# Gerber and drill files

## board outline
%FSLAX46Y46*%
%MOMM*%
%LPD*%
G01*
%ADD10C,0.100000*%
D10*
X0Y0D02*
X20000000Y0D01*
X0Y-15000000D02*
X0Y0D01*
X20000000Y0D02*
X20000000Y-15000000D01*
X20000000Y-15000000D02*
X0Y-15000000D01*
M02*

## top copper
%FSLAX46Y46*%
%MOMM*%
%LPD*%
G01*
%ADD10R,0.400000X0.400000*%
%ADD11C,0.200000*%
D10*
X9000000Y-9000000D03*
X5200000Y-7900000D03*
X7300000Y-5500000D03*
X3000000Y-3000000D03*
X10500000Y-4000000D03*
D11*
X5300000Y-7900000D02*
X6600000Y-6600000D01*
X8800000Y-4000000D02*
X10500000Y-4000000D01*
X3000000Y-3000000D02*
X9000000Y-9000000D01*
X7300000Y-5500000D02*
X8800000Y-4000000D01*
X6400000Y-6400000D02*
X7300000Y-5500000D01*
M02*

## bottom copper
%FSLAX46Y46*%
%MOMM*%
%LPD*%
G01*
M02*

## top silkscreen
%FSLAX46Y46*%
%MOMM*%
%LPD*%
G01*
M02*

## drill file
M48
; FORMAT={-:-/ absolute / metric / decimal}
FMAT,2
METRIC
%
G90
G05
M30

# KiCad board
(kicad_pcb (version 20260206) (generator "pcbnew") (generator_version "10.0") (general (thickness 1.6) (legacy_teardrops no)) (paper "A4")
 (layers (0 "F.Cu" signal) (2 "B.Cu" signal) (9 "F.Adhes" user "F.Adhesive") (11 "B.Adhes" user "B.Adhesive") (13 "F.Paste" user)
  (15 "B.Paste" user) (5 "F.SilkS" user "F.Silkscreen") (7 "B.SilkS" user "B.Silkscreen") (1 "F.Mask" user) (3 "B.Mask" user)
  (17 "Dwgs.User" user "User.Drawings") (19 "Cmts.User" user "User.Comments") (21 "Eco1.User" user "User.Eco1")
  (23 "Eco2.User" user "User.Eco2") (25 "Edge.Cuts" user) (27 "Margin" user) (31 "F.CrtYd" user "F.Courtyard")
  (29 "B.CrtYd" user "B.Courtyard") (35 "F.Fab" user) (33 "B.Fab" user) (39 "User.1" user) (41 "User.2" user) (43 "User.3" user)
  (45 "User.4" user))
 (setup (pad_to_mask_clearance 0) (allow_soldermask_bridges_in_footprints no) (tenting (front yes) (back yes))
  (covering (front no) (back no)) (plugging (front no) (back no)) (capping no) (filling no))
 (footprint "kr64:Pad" (layer "F.Cu") (at 9 9)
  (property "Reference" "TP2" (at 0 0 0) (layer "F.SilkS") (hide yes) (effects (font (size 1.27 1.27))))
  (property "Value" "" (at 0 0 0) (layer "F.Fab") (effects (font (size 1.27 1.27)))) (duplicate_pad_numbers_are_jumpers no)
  (pad "1" smd rect (at 0 0) (size 0.4 0.4) (layers "F.Cu" "F.Mask" "F.Paste") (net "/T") (thermal_bridge_angle 45)))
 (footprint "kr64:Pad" (layer "F.Cu") (at 5.2 7.9)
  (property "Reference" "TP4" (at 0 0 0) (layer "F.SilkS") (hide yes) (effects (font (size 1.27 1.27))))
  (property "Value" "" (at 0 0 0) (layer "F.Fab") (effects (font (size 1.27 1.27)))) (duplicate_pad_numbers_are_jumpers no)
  (pad "1" smd rect (at 0 0) (size 0.4 0.4) (layers "F.Cu" "F.Mask" "F.Paste") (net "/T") (thermal_bridge_angle 45)))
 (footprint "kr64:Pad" (layer "F.Cu") (at 7.3 5.5)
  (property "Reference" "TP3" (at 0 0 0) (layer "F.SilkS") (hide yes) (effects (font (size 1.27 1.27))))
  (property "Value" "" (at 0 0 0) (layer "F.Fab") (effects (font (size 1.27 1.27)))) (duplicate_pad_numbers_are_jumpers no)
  (pad "1" smd rect (at 0 0) (size 0.4 0.4) (layers "F.Cu" "F.Mask" "F.Paste") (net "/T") (thermal_bridge_angle 45)))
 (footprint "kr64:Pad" (layer "F.Cu") (at 3 3)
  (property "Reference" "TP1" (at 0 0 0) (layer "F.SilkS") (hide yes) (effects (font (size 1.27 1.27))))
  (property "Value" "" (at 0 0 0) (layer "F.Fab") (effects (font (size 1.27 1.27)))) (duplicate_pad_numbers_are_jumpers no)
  (pad "1" smd rect (at 0 0) (size 0.4 0.4) (layers "F.Cu" "F.Mask" "F.Paste") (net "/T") (thermal_bridge_angle 45)))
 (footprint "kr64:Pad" (layer "F.Cu") (at 10.5 4)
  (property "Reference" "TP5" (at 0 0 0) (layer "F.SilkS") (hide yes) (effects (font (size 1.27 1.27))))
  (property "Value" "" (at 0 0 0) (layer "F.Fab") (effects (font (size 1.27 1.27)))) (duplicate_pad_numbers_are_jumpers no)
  (pad "1" smd rect (at 0 0) (size 0.4 0.4) (layers "F.Cu" "F.Mask" "F.Paste") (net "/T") (thermal_bridge_angle 45)))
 (gr_line (start 0 0) (end 20 0) (stroke (width 0.1) (type default)) (layer "Edge.Cuts"))
 (gr_line (start 0 15) (end 0 0) (stroke (width 0.1) (type default)) (layer "Edge.Cuts"))
 (gr_line (start 20 0) (end 20 15) (stroke (width 0.1) (type default)) (layer "Edge.Cuts"))
 (gr_line (start 20 15) (end 0 15) (stroke (width 0.1) (type default)) (layer "Edge.Cuts"))
 (segment (start 5.3 7.9) (end 6.6 6.6) (width 0.2) (layer "F.Cu") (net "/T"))
 (segment (start 8.8 4) (end 10.5 4) (width 0.2) (layer "F.Cu") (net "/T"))
 (segment (start 3 3) (end 9 9) (width 0.2) (layer "F.Cu") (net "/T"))
 (segment (start 7.3 5.5) (end 8.8 4) (width 0.2) (layer "F.Cu") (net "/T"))
 (segment (start 6.4 6.4) (end 7.3 5.5) (width 0.2) (layer "F.Cu") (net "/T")))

